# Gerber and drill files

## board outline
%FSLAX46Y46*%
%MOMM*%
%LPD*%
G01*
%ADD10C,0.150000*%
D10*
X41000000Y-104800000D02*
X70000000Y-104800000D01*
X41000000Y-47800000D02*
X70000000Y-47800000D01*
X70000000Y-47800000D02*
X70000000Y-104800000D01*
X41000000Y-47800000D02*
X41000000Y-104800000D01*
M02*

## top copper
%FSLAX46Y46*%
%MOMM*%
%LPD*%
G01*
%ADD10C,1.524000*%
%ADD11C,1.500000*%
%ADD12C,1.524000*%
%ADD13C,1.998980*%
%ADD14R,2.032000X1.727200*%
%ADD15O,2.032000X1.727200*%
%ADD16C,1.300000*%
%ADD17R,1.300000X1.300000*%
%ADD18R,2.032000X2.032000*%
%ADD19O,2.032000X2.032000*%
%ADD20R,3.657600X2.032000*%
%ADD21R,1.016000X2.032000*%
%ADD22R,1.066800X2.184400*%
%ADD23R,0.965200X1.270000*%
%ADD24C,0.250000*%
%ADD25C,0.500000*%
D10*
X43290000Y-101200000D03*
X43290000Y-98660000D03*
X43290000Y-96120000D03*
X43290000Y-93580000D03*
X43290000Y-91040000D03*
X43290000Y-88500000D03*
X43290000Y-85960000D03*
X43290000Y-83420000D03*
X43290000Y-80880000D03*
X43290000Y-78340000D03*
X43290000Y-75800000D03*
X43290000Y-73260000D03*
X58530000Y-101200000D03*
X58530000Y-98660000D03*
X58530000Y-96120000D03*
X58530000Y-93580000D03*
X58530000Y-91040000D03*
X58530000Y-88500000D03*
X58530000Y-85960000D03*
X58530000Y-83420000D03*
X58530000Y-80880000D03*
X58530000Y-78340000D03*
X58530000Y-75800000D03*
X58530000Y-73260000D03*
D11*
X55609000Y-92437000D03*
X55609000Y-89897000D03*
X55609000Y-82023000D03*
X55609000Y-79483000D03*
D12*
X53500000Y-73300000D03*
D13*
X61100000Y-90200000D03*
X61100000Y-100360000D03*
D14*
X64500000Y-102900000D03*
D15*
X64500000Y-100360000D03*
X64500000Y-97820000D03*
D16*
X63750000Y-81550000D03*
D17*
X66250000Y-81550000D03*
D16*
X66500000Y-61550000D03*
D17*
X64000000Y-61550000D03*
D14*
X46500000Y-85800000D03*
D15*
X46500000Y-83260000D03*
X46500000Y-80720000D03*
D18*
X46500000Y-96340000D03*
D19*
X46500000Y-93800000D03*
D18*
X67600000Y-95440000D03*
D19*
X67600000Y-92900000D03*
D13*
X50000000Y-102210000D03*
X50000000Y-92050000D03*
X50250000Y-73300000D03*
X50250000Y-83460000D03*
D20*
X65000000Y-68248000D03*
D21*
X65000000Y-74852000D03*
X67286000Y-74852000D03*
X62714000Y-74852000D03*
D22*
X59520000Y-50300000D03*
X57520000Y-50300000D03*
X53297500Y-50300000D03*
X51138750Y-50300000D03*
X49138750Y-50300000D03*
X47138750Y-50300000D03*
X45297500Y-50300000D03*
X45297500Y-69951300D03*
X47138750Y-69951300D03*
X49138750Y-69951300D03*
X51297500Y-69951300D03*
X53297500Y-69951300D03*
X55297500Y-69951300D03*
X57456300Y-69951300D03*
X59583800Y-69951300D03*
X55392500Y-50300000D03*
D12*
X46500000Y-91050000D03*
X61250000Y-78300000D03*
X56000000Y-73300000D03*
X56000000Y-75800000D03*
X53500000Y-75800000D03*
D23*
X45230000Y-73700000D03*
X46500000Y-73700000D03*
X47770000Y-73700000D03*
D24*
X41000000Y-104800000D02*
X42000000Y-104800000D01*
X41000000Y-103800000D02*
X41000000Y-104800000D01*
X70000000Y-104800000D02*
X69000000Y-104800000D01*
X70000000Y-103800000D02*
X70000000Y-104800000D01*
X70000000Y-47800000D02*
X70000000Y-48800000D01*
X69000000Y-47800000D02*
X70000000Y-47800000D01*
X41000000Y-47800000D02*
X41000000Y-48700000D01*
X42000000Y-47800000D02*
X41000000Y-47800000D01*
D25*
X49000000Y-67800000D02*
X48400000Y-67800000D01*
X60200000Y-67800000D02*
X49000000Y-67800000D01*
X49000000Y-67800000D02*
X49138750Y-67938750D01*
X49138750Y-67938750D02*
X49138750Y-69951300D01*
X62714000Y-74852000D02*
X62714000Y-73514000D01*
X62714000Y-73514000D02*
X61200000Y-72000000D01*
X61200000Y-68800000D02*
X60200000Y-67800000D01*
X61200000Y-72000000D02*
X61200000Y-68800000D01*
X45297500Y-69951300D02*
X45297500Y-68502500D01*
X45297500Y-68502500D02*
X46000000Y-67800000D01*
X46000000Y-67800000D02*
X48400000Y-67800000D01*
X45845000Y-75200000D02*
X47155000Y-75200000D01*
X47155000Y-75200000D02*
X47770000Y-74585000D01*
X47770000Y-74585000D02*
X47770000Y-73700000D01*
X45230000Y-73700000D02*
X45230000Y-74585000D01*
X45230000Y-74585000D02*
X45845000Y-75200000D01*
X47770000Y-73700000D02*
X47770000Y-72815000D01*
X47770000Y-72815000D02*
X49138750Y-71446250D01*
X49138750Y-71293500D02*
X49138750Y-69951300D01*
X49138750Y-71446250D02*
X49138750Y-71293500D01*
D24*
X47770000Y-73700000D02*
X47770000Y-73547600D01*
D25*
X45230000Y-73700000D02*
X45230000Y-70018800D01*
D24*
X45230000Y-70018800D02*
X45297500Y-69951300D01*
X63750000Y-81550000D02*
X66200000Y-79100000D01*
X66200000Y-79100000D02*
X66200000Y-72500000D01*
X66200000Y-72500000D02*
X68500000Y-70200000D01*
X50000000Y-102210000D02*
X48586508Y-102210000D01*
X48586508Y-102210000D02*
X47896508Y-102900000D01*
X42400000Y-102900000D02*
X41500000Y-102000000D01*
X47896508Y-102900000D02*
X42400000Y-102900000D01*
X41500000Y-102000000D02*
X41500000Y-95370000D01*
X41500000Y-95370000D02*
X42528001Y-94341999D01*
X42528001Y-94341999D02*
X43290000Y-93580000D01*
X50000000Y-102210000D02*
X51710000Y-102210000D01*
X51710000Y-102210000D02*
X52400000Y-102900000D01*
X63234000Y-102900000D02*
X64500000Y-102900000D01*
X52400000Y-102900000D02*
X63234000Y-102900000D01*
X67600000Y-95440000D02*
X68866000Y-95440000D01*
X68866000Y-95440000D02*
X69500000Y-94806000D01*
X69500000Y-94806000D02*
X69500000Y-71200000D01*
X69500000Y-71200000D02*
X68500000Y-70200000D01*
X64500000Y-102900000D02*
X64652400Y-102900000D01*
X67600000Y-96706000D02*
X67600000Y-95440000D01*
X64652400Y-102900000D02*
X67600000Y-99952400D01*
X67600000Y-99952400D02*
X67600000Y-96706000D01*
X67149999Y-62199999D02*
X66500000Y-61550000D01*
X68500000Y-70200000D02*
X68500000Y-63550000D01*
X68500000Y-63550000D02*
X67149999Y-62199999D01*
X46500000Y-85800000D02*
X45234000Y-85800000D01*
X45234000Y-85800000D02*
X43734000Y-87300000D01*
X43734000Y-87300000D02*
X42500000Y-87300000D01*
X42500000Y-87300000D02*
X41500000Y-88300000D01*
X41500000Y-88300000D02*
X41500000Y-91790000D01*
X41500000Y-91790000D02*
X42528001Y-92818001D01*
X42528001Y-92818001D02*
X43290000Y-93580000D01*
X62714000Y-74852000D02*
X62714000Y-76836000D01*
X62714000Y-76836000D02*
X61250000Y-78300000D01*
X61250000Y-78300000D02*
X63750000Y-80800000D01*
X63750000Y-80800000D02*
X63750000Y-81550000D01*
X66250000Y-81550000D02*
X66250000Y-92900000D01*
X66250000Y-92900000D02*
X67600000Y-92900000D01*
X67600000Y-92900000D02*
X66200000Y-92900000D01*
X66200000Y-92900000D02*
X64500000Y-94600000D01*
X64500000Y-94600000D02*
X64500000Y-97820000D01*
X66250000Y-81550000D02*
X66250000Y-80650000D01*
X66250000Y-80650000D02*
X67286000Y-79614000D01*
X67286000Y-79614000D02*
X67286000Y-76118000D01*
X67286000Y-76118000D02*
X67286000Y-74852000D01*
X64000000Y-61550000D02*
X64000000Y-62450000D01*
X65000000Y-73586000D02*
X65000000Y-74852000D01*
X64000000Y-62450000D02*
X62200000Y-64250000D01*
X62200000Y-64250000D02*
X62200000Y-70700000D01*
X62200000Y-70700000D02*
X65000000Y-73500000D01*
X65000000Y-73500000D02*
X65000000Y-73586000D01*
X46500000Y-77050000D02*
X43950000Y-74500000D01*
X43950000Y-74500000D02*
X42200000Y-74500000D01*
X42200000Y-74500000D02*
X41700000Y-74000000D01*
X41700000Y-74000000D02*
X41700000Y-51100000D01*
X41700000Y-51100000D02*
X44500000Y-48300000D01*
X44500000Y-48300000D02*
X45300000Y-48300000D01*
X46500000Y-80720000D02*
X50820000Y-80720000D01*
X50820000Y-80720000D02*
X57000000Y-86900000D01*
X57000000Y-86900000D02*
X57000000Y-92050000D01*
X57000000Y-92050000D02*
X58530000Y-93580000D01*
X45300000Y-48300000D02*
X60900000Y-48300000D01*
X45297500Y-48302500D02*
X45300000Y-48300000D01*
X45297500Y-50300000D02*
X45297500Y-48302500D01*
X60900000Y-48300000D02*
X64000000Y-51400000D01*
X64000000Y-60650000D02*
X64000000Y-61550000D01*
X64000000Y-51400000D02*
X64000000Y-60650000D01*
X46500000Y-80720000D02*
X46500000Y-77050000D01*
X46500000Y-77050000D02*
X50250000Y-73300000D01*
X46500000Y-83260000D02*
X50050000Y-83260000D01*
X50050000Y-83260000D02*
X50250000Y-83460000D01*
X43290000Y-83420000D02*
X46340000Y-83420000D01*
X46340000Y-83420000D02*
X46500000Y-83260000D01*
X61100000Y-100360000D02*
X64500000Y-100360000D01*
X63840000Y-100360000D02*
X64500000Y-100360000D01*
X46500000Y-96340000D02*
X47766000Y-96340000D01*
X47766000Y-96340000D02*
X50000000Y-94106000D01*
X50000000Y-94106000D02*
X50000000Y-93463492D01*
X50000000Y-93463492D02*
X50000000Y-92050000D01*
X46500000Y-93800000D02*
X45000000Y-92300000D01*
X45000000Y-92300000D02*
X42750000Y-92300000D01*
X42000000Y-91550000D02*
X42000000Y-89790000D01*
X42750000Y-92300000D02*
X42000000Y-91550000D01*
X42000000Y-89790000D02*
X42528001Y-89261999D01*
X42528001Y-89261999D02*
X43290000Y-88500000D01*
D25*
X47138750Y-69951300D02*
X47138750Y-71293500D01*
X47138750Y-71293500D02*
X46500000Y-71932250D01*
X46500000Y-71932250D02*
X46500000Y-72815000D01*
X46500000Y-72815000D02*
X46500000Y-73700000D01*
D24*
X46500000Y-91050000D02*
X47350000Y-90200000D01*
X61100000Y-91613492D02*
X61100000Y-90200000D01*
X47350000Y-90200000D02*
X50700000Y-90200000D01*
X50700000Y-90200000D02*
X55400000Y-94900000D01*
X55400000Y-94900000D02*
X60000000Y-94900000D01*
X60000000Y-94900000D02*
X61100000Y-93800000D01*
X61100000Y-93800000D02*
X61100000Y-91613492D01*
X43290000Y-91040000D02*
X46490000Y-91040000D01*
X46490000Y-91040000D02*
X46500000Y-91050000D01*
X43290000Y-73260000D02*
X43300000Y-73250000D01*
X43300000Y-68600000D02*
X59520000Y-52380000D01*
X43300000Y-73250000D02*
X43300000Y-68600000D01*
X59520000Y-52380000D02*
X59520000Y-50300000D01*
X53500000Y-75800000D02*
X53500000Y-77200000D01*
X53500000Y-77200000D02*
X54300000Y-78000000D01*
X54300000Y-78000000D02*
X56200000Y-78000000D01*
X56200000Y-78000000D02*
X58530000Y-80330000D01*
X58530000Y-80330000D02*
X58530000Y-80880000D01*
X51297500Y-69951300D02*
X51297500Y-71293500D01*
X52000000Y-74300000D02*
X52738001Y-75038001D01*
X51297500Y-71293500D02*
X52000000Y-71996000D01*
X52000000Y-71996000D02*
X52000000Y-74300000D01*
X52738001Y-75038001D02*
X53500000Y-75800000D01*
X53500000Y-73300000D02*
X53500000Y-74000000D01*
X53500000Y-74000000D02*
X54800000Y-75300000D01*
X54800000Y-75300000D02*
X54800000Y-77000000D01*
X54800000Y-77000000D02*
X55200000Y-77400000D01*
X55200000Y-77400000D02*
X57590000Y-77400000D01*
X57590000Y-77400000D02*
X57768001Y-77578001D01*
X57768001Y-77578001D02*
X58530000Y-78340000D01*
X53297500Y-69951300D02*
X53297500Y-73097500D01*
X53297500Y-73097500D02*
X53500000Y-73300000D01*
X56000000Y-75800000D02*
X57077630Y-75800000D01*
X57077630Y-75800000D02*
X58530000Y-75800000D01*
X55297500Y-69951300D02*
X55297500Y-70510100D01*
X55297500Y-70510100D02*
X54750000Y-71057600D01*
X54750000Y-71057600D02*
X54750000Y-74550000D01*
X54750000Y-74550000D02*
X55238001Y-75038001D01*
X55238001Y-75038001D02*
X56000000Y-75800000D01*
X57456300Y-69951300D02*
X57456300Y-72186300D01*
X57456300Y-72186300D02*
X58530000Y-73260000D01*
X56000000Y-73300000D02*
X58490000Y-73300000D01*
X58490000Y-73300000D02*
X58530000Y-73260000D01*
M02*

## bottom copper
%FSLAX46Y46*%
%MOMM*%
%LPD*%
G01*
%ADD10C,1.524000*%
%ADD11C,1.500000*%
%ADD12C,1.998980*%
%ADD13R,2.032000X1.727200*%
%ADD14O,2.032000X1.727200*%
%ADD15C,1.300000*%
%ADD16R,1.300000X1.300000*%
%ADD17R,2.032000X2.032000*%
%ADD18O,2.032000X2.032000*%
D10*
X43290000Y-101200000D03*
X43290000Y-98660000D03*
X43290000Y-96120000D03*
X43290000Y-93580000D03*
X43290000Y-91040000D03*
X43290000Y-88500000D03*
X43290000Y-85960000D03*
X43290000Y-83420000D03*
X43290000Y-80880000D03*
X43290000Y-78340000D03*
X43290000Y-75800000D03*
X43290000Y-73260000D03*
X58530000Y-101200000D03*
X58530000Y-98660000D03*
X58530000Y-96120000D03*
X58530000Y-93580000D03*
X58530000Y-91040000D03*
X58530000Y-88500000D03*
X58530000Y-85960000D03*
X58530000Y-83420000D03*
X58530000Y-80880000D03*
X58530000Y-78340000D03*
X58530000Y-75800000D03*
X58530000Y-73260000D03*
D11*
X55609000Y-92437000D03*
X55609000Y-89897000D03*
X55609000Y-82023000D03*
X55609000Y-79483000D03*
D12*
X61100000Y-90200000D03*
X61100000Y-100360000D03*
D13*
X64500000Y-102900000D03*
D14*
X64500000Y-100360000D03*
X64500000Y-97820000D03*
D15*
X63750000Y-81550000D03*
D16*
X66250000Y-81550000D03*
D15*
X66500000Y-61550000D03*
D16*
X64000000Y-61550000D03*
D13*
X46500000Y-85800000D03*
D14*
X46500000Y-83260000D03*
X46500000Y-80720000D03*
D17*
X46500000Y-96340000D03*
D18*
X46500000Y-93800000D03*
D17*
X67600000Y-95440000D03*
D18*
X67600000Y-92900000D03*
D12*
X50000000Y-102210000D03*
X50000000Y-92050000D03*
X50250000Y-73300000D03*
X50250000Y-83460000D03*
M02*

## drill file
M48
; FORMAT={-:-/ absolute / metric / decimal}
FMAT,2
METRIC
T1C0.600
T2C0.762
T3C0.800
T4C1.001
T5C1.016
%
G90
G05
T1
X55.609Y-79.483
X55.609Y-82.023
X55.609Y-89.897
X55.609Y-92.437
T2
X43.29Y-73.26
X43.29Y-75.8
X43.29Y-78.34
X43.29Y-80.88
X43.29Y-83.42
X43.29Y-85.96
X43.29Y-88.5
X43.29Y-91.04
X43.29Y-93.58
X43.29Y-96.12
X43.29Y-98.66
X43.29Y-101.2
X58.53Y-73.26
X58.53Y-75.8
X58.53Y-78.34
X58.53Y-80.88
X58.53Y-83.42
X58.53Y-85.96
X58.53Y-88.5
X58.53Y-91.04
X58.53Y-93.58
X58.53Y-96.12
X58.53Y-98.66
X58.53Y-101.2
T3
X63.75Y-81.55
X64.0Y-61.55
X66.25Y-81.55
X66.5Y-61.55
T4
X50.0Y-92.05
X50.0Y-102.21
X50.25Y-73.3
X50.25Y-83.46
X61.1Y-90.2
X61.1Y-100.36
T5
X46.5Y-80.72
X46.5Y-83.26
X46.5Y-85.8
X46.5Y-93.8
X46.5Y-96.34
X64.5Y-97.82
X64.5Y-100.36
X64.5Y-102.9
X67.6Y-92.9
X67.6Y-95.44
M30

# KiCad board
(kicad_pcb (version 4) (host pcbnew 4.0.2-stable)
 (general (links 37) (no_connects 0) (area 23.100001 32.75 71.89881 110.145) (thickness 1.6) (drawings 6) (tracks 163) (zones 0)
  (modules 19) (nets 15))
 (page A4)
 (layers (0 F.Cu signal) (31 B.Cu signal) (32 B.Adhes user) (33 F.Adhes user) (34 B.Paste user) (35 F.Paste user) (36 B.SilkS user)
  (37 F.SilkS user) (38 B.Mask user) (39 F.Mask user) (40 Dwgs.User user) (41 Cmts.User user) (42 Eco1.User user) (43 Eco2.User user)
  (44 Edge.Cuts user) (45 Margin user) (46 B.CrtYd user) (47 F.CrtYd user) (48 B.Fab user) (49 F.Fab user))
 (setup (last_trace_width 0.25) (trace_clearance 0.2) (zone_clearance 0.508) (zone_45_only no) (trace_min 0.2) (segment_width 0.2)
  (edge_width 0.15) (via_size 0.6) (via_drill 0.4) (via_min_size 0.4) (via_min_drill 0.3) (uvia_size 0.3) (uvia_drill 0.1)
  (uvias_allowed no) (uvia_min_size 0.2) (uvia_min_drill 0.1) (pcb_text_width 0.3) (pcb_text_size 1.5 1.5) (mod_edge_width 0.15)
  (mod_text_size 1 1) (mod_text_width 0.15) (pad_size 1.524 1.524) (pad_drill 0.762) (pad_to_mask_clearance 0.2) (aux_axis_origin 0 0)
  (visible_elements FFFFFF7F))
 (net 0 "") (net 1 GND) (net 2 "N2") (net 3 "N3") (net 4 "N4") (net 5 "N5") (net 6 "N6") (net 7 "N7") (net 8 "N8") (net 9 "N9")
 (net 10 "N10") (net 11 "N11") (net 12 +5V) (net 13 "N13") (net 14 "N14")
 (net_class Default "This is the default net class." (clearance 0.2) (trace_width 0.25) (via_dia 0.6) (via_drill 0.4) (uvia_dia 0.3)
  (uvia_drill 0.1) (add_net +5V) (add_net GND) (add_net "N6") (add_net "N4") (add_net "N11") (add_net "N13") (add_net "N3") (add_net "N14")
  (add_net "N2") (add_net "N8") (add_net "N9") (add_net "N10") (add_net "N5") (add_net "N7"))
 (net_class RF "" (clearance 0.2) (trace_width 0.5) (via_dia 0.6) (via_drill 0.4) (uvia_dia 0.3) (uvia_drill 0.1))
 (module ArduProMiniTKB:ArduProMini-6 (layer B.Cu) (at 40.75 107.55)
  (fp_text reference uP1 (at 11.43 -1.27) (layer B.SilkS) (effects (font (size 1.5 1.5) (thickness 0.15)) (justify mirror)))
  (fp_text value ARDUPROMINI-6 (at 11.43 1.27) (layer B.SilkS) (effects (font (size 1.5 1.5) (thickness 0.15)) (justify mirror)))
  (pad 7 thru_hole circle (at 2.54 -6.35) (size 1.524 1.524) (drill 0.762) (layers *.Cu *.Mask B.SilkS))
  (pad 8 thru_hole circle (at 2.54 -8.89) (size 1.524 1.524) (drill 0.762) (layers *.Cu *.Mask B.SilkS))
  (pad 9 thru_hole circle (at 2.54 -11.43) (size 1.524 1.524) (drill 0.762) (layers *.Cu *.Mask B.SilkS))
  (pad 10 thru_hole circle (at 2.54 -13.97) (size 1.524 1.524) (drill 0.762) (layers *.Cu *.Mask B.SilkS) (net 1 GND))
  (pad 11 thru_hole circle (at 2.54 -16.51) (size 1.524 1.524) (drill 0.762) (layers *.Cu *.Mask B.SilkS) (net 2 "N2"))
  (pad 12 thru_hole circle (at 2.54 -19.05) (size 1.524 1.524) (drill 0.762) (layers *.Cu *.Mask B.SilkS) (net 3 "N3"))
  (pad 13 thru_hole circle (at 2.54 -21.59) (size 1.524 1.524) (drill 0.762) (layers *.Cu *.Mask B.SilkS))
  (pad 14 thru_hole circle (at 2.54 -24.13) (size 1.524 1.524) (drill 0.762) (layers *.Cu *.Mask B.SilkS) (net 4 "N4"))
  (pad 15 thru_hole circle (at 2.54 -26.67) (size 1.524 1.524) (drill 0.762) (layers *.Cu *.Mask B.SilkS))
  (pad 16 thru_hole circle (at 2.54 -29.21) (size 1.524 1.524) (drill 0.762) (layers *.Cu *.Mask B.SilkS))
  (pad 17 thru_hole circle (at 2.54 -31.75) (size 1.524 1.524) (drill 0.762) (layers *.Cu *.Mask B.SilkS))
  (pad 18 thru_hole circle (at 2.54 -34.29) (size 1.524 1.524) (drill 0.762) (layers *.Cu *.Mask B.SilkS) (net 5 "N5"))
  (pad 19 thru_hole circle (at 17.78 -6.35) (size 1.524 1.524) (drill 0.762) (layers *.Cu *.Mask B.SilkS))
  (pad 20 thru_hole circle (at 17.78 -8.89) (size 1.524 1.524) (drill 0.762) (layers *.Cu *.Mask B.SilkS))
  (pad 21 thru_hole circle (at 17.78 -11.43) (size 1.524 1.524) (drill 0.762) (layers *.Cu *.Mask B.SilkS))
  (pad 22 thru_hole circle (at 17.78 -13.97) (size 1.524 1.524) (drill 0.762) (layers *.Cu *.Mask B.SilkS) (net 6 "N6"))
  (pad 23 thru_hole circle (at 17.78 -16.51) (size 1.524 1.524) (drill 0.762) (layers *.Cu *.Mask B.SilkS))
  (pad 24 thru_hole circle (at 17.78 -19.05) (size 1.524 1.524) (drill 0.762) (layers *.Cu *.Mask B.SilkS))
  (pad 25 thru_hole circle (at 17.78 -21.59) (size 1.524 1.524) (drill 0.762) (layers *.Cu *.Mask B.SilkS))
  (pad 26 thru_hole circle (at 17.78 -24.13) (size 1.524 1.524) (drill 0.762) (layers *.Cu *.Mask B.SilkS))
  (pad 27 thru_hole circle (at 17.78 -26.67) (size 1.524 1.524) (drill 0.762) (layers *.Cu *.Mask B.SilkS) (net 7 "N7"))
  (pad 28 thru_hole circle (at 17.78 -29.21) (size 1.524 1.524) (drill 0.762) (layers *.Cu *.Mask B.SilkS) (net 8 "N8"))
  (pad 29 thru_hole circle (at 17.78 -31.75) (size 1.524 1.524) (drill 0.762) (layers *.Cu *.Mask B.SilkS) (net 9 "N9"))
  (pad 30 thru_hole circle (at 17.78 -34.29) (size 1.524 1.524) (drill 0.762) (layers *.Cu *.Mask B.SilkS) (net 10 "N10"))
  (pad 31 thru_hole circle (at 14.859 -15.113) (size 1.5 1.5) (drill 0.6) (layers *.Cu *.Mask B.SilkS))
  (pad 32 thru_hole circle (at 14.859 -17.653) (size 1.5 1.5) (drill 0.6) (layers *.Cu *.Mask B.SilkS))
  (pad 34 thru_hole circle (at 14.859 -25.527) (size 1.5 1.5) (drill 0.6) (layers *.Cu *.Mask B.SilkS))
  (pad 35 thru_hole circle (at 14.859 -28.067) (size 1.5 1.5) (drill 0.6) (layers *.Cu *.Mask B.SilkS)))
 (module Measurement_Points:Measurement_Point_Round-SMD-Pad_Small (layer F.Cu) (at 53.5 73.3)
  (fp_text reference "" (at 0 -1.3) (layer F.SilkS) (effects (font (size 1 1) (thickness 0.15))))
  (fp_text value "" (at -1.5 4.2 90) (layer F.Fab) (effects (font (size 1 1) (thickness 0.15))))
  (pad 1 smd circle (at 0 0) (size 1.524 1.524) (layers F.Cu F.Paste F.Mask) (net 8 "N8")))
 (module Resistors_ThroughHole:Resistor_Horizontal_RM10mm (layer F.Cu) (at 61.1 90.2 270)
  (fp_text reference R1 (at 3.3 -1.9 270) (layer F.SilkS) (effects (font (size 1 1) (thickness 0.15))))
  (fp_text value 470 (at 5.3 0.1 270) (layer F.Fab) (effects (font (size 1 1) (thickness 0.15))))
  (pad 1 thru_hole circle (at 0 0 270) (size 1.99898 1.99898) (drill 1.00076) (layers *.Cu *.SilkS *.Mask) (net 2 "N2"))
  (pad 2 thru_hole circle (at 10.16 0 270) (size 1.99898 1.99898) (drill 1.00076) (layers *.Cu *.SilkS *.Mask) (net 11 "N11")))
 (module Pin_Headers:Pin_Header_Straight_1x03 (layer F.Cu) (at 64.5 102.9 180)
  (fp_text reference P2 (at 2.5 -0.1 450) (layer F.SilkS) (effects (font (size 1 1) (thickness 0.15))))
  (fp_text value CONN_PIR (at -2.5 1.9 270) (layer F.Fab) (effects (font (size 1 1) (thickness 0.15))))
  (pad 1 thru_hole rect (at 0 0 180) (size 2.032 1.7272) (drill 1.016) (layers *.Cu *.Mask F.SilkS) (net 1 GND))
  (pad 2 thru_hole oval (at 0 2.54 180) (size 2.032 1.7272) (drill 1.016) (layers *.Cu *.Mask F.SilkS) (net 11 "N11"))
  (pad 3 thru_hole oval (at 0 5.08 180) (size 2.032 1.7272) (drill 1.016) (layers *.Cu *.Mask F.SilkS) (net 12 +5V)))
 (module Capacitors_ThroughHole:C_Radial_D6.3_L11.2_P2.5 (layer F.Cu) (at 66.25 81.55 180)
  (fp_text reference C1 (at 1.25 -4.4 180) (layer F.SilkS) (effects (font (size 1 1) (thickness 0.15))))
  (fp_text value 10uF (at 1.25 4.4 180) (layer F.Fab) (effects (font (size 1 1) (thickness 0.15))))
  (pad 2 thru_hole circle (at 2.5 0 180) (size 1.3 1.3) (drill 0.8) (layers *.Cu *.Mask F.SilkS) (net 1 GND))
  (pad 1 thru_hole rect (at 0 0 180) (size 1.3 1.3) (drill 0.8) (layers *.Cu *.Mask F.SilkS) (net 12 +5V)))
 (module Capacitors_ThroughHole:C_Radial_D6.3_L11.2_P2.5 (layer F.Cu) (at 64 61.55)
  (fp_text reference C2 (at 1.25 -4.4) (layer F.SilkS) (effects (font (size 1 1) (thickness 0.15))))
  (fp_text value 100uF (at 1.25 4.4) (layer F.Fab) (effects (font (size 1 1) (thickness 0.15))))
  (pad 2 thru_hole circle (at 2.5 0) (size 1.3 1.3) (drill 0.8) (layers *.Cu *.Mask F.SilkS) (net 1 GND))
  (pad 1 thru_hole rect (at 0 0) (size 1.3 1.3) (drill 0.8) (layers *.Cu *.Mask F.SilkS) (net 6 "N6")))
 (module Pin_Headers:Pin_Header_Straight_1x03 (layer F.Cu) (at 46.5 85.8 180)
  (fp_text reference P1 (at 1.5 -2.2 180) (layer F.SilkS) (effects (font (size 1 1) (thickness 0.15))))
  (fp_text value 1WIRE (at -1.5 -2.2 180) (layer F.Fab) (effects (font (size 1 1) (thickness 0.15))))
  (pad 1 thru_hole rect (at 0 0 180) (size 2.032 1.7272) (drill 1.016) (layers *.Cu *.Mask F.SilkS) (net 1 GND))
  (pad 2 thru_hole oval (at 0 2.54 180) (size 2.032 1.7272) (drill 1.016) (layers *.Cu *.Mask F.SilkS) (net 4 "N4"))
  (pad 3 thru_hole oval (at 0 5.08 180) (size 2.032 1.7272) (drill 1.016) (layers *.Cu *.Mask F.SilkS) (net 6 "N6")))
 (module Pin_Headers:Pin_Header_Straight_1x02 (layer F.Cu) (at 46.5 96.34 180)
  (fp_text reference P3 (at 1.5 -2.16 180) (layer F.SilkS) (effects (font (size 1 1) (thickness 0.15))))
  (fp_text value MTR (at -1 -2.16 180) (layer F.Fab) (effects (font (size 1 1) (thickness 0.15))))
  (pad 1 thru_hole rect (at 0 0 180) (size 2.032 2.032) (drill 1.016) (layers *.Cu *.Mask F.SilkS) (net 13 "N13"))
  (pad 2 thru_hole oval (at 0 2.54 180) (size 2.032 2.032) (drill 1.016) (layers *.Cu *.Mask F.SilkS) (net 3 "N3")))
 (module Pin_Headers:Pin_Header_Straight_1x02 (layer F.Cu) (at 67.6 95.44 180)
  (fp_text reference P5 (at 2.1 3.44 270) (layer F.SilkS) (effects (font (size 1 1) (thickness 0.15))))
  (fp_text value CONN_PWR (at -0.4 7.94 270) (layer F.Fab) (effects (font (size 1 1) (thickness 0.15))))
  (pad 1 thru_hole rect (at 0 0 180) (size 2.032 2.032) (drill 1.016) (layers *.Cu *.Mask F.SilkS) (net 1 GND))
  (pad 2 thru_hole oval (at 0 2.54 180) (size 2.032 2.032) (drill 1.016) (layers *.Cu *.Mask F.SilkS) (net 12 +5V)))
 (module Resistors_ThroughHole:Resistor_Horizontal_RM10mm (layer F.Cu) (at 50 102.21 90)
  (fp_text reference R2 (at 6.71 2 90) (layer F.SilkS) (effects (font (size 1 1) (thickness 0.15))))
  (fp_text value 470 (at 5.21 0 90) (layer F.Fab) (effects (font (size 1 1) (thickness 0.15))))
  (pad 1 thru_hole circle (at 0 0 90) (size 1.99898 1.99898) (drill 1.00076) (layers *.Cu *.SilkS *.Mask) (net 1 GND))
  (pad 2 thru_hole circle (at 10.16 0 90) (size 1.99898 1.99898) (drill 1.00076) (layers *.Cu *.SilkS *.Mask) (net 13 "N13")))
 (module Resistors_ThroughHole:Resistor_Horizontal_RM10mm (layer F.Cu) (at 50.25 73.3 270)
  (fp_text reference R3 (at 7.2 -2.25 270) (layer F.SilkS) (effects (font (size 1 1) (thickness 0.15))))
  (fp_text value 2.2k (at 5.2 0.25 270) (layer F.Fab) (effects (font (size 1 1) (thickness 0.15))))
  (pad 1 thru_hole circle (at 0 0 270) (size 1.99898 1.99898) (drill 1.00076) (layers *.Cu *.SilkS *.Mask) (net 6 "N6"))
  (pad 2 thru_hole circle (at 10.16 0 270) (size 1.99898 1.99898) (drill 1.00076) (layers *.Cu *.SilkS *.Mask) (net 4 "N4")))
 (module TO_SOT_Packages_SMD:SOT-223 (layer F.Cu) (at 65 71.55)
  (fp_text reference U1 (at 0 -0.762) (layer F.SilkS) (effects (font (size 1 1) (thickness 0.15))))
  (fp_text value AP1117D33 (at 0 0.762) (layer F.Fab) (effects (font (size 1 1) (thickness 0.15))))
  (pad 4 smd rect (at 0 -3.302) (size 3.6576 2.032) (layers F.Cu F.Paste F.Mask))
  (pad 2 smd rect (at 0 3.302) (size 1.016 2.032) (layers F.Cu F.Paste F.Mask) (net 6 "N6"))
  (pad 3 smd rect (at 2.286 3.302) (size 1.016 2.032) (layers F.Cu F.Paste F.Mask) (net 12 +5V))
  (pad 1 smd rect (at -2.286 3.302) (size 1.016 2.032) (layers F.Cu F.Paste F.Mask) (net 1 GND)))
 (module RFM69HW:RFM (layer F.Cu) (at 44.25 50.3 270) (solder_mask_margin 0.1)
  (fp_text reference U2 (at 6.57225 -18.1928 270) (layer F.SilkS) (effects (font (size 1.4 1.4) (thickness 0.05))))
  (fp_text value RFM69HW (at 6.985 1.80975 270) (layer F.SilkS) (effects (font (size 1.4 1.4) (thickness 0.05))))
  (pad RESE smd rect (at 0 -15.27 270) (size 2.1844 1.0668) (layers F.Cu F.Paste F.Mask) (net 5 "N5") (solder_mask_margin 0.2))
  (pad DIO0 smd rect (at 0 -13.27 270) (size 2.1844 1.0668) (layers F.Cu F.Paste F.Mask) (solder_mask_margin 0.2))
  (pad DIO2 smd rect (at 0 -9.0475 270) (size 2.1844 1.0668) (layers F.Cu F.Paste F.Mask) (solder_mask_margin 0.2))
  (pad DIO3 smd rect (at 0 -6.88875 270) (size 2.1844 1.0668) (layers F.Cu F.Paste F.Mask) (solder_mask_margin 0.2))
  (pad DIO4 smd rect (at 0 -4.88875 270) (size 2.1844 1.0668) (layers F.Cu F.Paste F.Mask) (solder_mask_margin 0.2))
  (pad DIO5 smd rect (at 0 -2.88875 270) (size 2.1844 1.0668) (layers F.Cu F.Paste F.Mask) (solder_mask_margin 0.2))
  (pad VCC smd rect (at 0 -1.0475 270) (size 2.1844 1.0668) (layers F.Cu F.Paste F.Mask) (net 6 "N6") (solder_mask_margin 0.2))
  (pad GNDB smd rect (at 19.6513 -1.0475 270) (size 2.1844 1.0668) (layers F.Cu F.Paste F.Mask) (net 1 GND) (solder_mask_margin 0.2))
  (pad ANT smd rect (at 19.6513 -2.88875 270) (size 2.1844 1.0668) (layers F.Cu F.Paste F.Mask) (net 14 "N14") (solder_mask_margin 0.2))
  (pad GNDA smd rect (at 19.6513 -4.88875 270) (size 2.1844 1.0668) (layers F.Cu F.Paste F.Mask) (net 1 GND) (solder_mask_margin 0.2))
  (pad SCK smd rect (at 19.6513 -7.0475 270) (size 2.1844 1.0668) (layers F.Cu F.Paste F.Mask) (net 7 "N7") (solder_mask_margin 0.2))
  (pad MISO smd rect (at 19.6513 -9.0475 270) (size 2.1844 1.0668) (layers F.Cu F.Paste F.Mask) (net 8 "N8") (solder_mask_margin 0.2))
  (pad MOSI smd rect (at 19.6513 -11.0475 270) (size 2.1844 1.0668) (layers F.Cu F.Paste F.Mask) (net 9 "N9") (solder_mask_margin 0.2))
  (pad NSS smd rect (at 19.6513 -13.2063 270) (size 2.1844 1.0668) (layers F.Cu F.Paste F.Mask) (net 10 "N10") (solder_mask_margin 0.2))
  (pad NC smd rect (at 19.6513 -15.3338 270) (size 2.1844 1.0668) (layers F.Cu F.Paste F.Mask) (solder_mask_margin 0.2))
  (pad DIO1 smd rect (at 0 -11.1425 270) (size 2.1844 1.0668) (layers F.Cu F.Paste F.Mask) (solder_mask_margin 0.2)))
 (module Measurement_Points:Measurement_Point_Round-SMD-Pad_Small (layer F.Cu) (at 46.5 91.05)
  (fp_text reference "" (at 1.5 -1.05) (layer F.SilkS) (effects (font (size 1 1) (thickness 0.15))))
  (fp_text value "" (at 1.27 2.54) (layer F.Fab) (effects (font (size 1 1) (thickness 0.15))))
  (pad 1 smd circle (at 0 0) (size 1.524 1.524) (layers F.Cu F.Paste F.Mask) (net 2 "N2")))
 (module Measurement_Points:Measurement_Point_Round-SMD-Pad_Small (layer F.Cu) (at 61.25 78.3)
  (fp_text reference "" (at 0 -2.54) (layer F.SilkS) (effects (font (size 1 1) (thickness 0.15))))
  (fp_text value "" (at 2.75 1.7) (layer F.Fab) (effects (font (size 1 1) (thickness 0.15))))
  (pad 1 smd circle (at 0 0) (size 1.524 1.524) (layers F.Cu F.Paste F.Mask) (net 1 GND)))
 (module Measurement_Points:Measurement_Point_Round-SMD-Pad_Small (layer F.Cu) (at 56 73.3)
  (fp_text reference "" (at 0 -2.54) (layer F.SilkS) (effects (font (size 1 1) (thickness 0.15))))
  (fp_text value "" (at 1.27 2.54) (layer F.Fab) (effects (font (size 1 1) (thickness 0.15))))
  (pad 1 smd circle (at 0 0) (size 1.524 1.524) (layers F.Cu F.Paste F.Mask) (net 10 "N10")))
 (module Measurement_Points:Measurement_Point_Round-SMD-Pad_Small (layer F.Cu) (at 56 75.8)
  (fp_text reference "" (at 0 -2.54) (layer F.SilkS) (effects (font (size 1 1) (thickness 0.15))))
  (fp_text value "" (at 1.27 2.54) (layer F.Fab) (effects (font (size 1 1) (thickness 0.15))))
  (pad 1 smd circle (at 0 0) (size 1.524 1.524) (layers F.Cu F.Paste F.Mask) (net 9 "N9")))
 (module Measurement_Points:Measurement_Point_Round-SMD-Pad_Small (layer F.Cu) (at 53.5 75.8)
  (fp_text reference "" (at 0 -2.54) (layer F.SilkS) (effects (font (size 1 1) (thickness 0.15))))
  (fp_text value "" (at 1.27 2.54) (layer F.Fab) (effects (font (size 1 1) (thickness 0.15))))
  (pad 1 smd circle (at 0 0) (size 1.524 1.524) (layers F.Cu F.Paste F.Mask) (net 7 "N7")))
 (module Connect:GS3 (layer F.Cu) (at 46.5 73.7 90)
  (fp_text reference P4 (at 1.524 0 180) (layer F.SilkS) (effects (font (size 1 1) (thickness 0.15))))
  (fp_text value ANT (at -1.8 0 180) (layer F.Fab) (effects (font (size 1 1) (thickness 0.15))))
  (pad 1 smd rect (at 0 -1.27 90) (size 1.27 0.9652) (layers F.Cu F.Paste F.Mask) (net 1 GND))
  (pad 2 smd rect (at 0 0 90) (size 1.27 0.9652) (layers F.Cu F.Paste F.Mask) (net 14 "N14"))
  (pad 3 smd rect (at 0 1.27 90) (size 1.27 0.9652) (layers F.Cu F.Paste F.Mask) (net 1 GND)))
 (gr_line (start 41 104.8) (end 70 104.8) (angle 90) (layer Edge.Cuts) (width 0.15))
 (gr_line (start 41 47.8) (end 70 47.8) (angle 90) (layer Edge.Cuts) (width 0.15))
 (gr_line (start 70 47.8) (end 70 104.8) (angle 90) (layer Edge.Cuts) (width 0.15))
 (gr_line (start 41 47.8) (end 41 104.8) (angle 90) (layer Edge.Cuts) (width 0.15))
 (segment (start 41 104.8) (end 42 104.8) (width 0.25) (layer F.Cu) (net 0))
 (segment (start 41 103.8) (end 41 104.8) (width 0.25) (layer F.Cu) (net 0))
 (segment (start 70 104.8) (end 69 104.8) (width 0.25) (layer F.Cu) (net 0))
 (segment (start 70 103.8) (end 70 104.8) (width 0.25) (layer F.Cu) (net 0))
 (segment (start 70 47.8) (end 70 48.8) (width 0.25) (layer F.Cu) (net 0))
 (segment (start 69 47.8) (end 70 47.8) (width 0.25) (layer F.Cu) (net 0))
 (segment (start 41 47.8) (end 41 48.7) (width 0.25) (layer F.Cu) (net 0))
 (segment (start 42 47.8) (end 41 47.8) (width 0.25) (layer F.Cu) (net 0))
 (segment (start 49 67.8) (end 48.4 67.8) (width 0.5) (layer F.Cu) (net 1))
 (segment (start 60.2 67.8) (end 49 67.8) (width 0.5) (layer F.Cu) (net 1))
 (segment (start 49 67.8) (end 49.13875 67.93875) (width 0.5) (layer F.Cu) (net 1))
 (segment (start 49.13875 67.93875) (end 49.13875 69.9513) (width 0.5) (layer F.Cu) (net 1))
 (segment (start 62.714 74.852) (end 62.714 73.514) (width 0.5) (layer F.Cu) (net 1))
 (segment (start 62.714 73.514) (end 61.2 72) (width 0.5) (layer F.Cu) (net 1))
 (segment (start 61.2 68.8) (end 60.2 67.8) (width 0.5) (layer F.Cu) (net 1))
 (segment (start 61.2 72) (end 61.2 68.8) (width 0.5) (layer F.Cu) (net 1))
 (segment (start 45.2975 69.9513) (end 45.2975 68.5025) (width 0.5) (layer F.Cu) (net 1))
 (segment (start 45.2975 68.5025) (end 46 67.8) (width 0.5) (layer F.Cu) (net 1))
 (segment (start 46 67.8) (end 48.4 67.8) (width 0.5) (layer F.Cu) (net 1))
 (segment (start 45.845 75.2) (end 47.155 75.2) (width 0.5) (layer F.Cu) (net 1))
 (segment (start 47.155 75.2) (end 47.77 74.585) (width 0.5) (layer F.Cu) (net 1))
 (segment (start 47.77 74.585) (end 47.77 73.7) (width 0.5) (layer F.Cu) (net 1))
 (segment (start 45.23 73.7) (end 45.23 74.585) (width 0.5) (layer F.Cu) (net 1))
 (segment (start 45.23 74.585) (end 45.845 75.2) (width 0.5) (layer F.Cu) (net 1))
 (segment (start 47.77 73.7) (end 47.77 72.815) (width 0.5) (layer F.Cu) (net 1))
 (segment (start 47.77 72.815) (end 49.13875 71.44625) (width 0.5) (layer F.Cu) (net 1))
 (segment (start 49.13875 71.2935) (end 49.13875 69.9513) (width 0.5) (layer F.Cu) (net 1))
 (segment (start 49.13875 71.44625) (end 49.13875 71.2935) (width 0.5) (layer F.Cu) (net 1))
 (segment (start 47.77 73.7) (end 47.77 73.5476) (width 0.25) (layer F.Cu) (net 1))
 (segment (start 45.23 73.7) (end 45.23 70.0188) (width 0.5) (layer F.Cu) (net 1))
 (segment (start 45.23 70.0188) (end 45.2975 69.9513) (width 0.25) (layer F.Cu) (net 1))
 (segment (start 63.75 81.55) (end 66.2 79.1) (width 0.25) (layer F.Cu) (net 1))
 (segment (start 66.2 79.1) (end 66.2 72.5) (width 0.25) (layer F.Cu) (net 1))
 (segment (start 66.2 72.5) (end 68.5 70.2) (width 0.25) (layer F.Cu) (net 1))
 (segment (start 50 102.21) (end 48.586508 102.21) (width 0.25) (layer F.Cu) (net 1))
 (segment (start 48.586508 102.21) (end 47.896508 102.9) (width 0.25) (layer F.Cu) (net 1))
 (segment (start 42.4 102.9) (end 41.5 102) (width 0.25) (layer F.Cu) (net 1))
 (segment (start 47.896508 102.9) (end 42.4 102.9) (width 0.25) (layer F.Cu) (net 1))
 (segment (start 41.5 102) (end 41.5 95.37) (width 0.25) (layer F.Cu) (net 1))
 (segment (start 41.5 95.37) (end 42.528001 94.341999) (width 0.25) (layer F.Cu) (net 1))
 (segment (start 42.528001 94.341999) (end 43.29 93.58) (width 0.25) (layer F.Cu) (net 1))
 (segment (start 50 102.21) (end 51.71 102.21) (width 0.25) (layer F.Cu) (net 1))
 (segment (start 51.71 102.21) (end 52.4 102.9) (width 0.25) (layer F.Cu) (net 1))
 (segment (start 63.234 102.9) (end 64.5 102.9) (width 0.25) (layer F.Cu) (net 1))
 (segment (start 52.4 102.9) (end 63.234 102.9) (width 0.25) (layer F.Cu) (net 1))
 (segment (start 67.6 95.44) (end 68.866 95.44) (width 0.25) (layer F.Cu) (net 1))
 (segment (start 68.866 95.44) (end 69.5 94.806) (width 0.25) (layer F.Cu) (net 1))
 (segment (start 69.5 94.806) (end 69.5 71.2) (width 0.25) (layer F.Cu) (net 1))
 (segment (start 69.5 71.2) (end 68.5 70.2) (width 0.25) (layer F.Cu) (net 1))
 (segment (start 64.5 102.9) (end 64.6524 102.9) (width 0.25) (layer F.Cu) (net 1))
 (segment (start 67.6 96.706) (end 67.6 95.44) (width 0.25) (layer F.Cu) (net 1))
 (segment (start 64.6524 102.9) (end 67.6 99.9524) (width 0.25) (layer F.Cu) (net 1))
 (segment (start 67.6 99.9524) (end 67.6 96.706) (width 0.25) (layer F.Cu) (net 1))
 (segment (start 67.149999 62.199999) (end 66.5 61.55) (width 0.25) (layer F.Cu) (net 1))
 (segment (start 68.5 70.2) (end 68.5 63.55) (width 0.25) (layer F.Cu) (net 1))
 (segment (start 68.5 63.55) (end 67.149999 62.199999) (width 0.25) (layer F.Cu) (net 1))
 (segment (start 46.5 85.8) (end 45.234 85.8) (width 0.25) (layer F.Cu) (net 1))
 (segment (start 45.234 85.8) (end 43.734 87.3) (width 0.25) (layer F.Cu) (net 1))
 (segment (start 43.734 87.3) (end 42.5 87.3) (width 0.25) (layer F.Cu) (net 1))
 (segment (start 42.5 87.3) (end 41.5 88.3) (width 0.25) (layer F.Cu) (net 1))
 (segment (start 41.5 88.3) (end 41.5 91.79) (width 0.25) (layer F.Cu) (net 1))
 (segment (start 41.5 91.79) (end 42.528001 92.818001) (width 0.25) (layer F.Cu) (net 1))
 (segment (start 42.528001 92.818001) (end 43.29 93.58) (width 0.25) (layer F.Cu) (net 1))
 (segment (start 62.714 74.852) (end 62.714 76.836) (width 0.25) (layer F.Cu) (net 1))
 (segment (start 62.714 76.836) (end 61.25 78.3) (width 0.25) (layer F.Cu) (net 1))
 (segment (start 61.25 78.3) (end 63.75 80.8) (width 0.25) (layer F.Cu) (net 1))
 (segment (start 63.75 80.8) (end 63.75 81.55) (width 0.25) (layer F.Cu) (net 1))
 (segment (start 66.25 81.55) (end 66.25 92.9) (width 0.25) (layer F.Cu) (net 12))
 (segment (start 66.25 92.9) (end 67.6 92.9) (width 0.25) (layer F.Cu) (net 12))
 (segment (start 67.6 92.9) (end 66.2 92.9) (width 0.25) (layer F.Cu) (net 12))
 (segment (start 66.2 92.9) (end 64.5 94.6) (width 0.25) (layer F.Cu) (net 12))
 (segment (start 64.5 94.6) (end 64.5 97.82) (width 0.25) (layer F.Cu) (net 12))
 (segment (start 66.25 81.55) (end 66.25 80.65) (width 0.25) (layer F.Cu) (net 12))
 (segment (start 66.25 80.65) (end 67.286 79.614) (width 0.25) (layer F.Cu) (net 12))
 (segment (start 67.286 79.614) (end 67.286 76.118) (width 0.25) (layer F.Cu) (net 12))
 (segment (start 67.286 76.118) (end 67.286 74.852) (width 0.25) (layer F.Cu) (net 12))
 (segment (start 64 61.55) (end 64 62.45) (width 0.25) (layer F.Cu) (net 6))
 (segment (start 65 73.586) (end 65 74.852) (width 0.25) (layer F.Cu) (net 6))
 (segment (start 64 62.45) (end 62.2 64.25) (width 0.25) (layer F.Cu) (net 6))
 (segment (start 62.2 64.25) (end 62.2 70.7) (width 0.25) (layer F.Cu) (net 6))
 (segment (start 62.2 70.7) (end 65 73.5) (width 0.25) (layer F.Cu) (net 6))
 (segment (start 65 73.5) (end 65 73.586) (width 0.25) (layer F.Cu) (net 6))
 (segment (start 46.5 77.05) (end 43.95 74.5) (width 0.25) (layer F.Cu) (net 6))
 (segment (start 43.95 74.5) (end 42.2 74.5) (width 0.25) (layer F.Cu) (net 6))
 (segment (start 42.2 74.5) (end 41.7 74) (width 0.25) (layer F.Cu) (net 6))
 (segment (start 41.7 74) (end 41.7 51.1) (width 0.25) (layer F.Cu) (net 6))
 (segment (start 41.7 51.1) (end 44.5 48.3) (width 0.25) (layer F.Cu) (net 6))
 (segment (start 44.5 48.3) (end 45.3 48.3) (width 0.25) (layer F.Cu) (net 6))
 (segment (start 46.5 80.72) (end 50.82 80.72) (width 0.25) (layer F.Cu) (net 6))
 (segment (start 50.82 80.72) (end 57 86.9) (width 0.25) (layer F.Cu) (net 6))
 (segment (start 57 86.9) (end 57 92.05) (width 0.25) (layer F.Cu) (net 6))
 (segment (start 57 92.05) (end 58.53 93.58) (width 0.25) (layer F.Cu) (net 6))
 (segment (start 45.3 48.3) (end 60.9 48.3) (width 0.25) (layer F.Cu) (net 6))
 (segment (start 45.2975 48.3025) (end 45.3 48.3) (width 0.25) (layer F.Cu) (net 6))
 (segment (start 45.2975 50.3) (end 45.2975 48.3025) (width 0.25) (layer F.Cu) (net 6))
 (segment (start 60.9 48.3) (end 64 51.4) (width 0.25) (layer F.Cu) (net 6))
 (segment (start 64 60.65) (end 64 61.55) (width 0.25) (layer F.Cu) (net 6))
 (segment (start 64 51.4) (end 64 60.65) (width 0.25) (layer F.Cu) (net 6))
 (segment (start 46.5 80.72) (end 46.5 77.05) (width 0.25) (layer F.Cu) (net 6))
 (segment (start 46.5 77.05) (end 50.25 73.3) (width 0.25) (layer F.Cu) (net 6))
 (segment (start 46.5 83.26) (end 50.05 83.26) (width 0.25) (layer F.Cu) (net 4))
 (segment (start 50.05 83.26) (end 50.25 83.46) (width 0.25) (layer F.Cu) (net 4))
 (segment (start 43.29 83.42) (end 46.34 83.42) (width 0.25) (layer F.Cu) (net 4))
 (segment (start 46.34 83.42) (end 46.5 83.26) (width 0.25) (layer F.Cu) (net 4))
 (segment (start 61.1 100.36) (end 64.5 100.36) (width 0.25) (layer F.Cu) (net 11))
 (segment (start 63.84 100.36) (end 64.5 100.36) (width 0.25) (layer F.Cu) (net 11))
 (segment (start 46.5 96.34) (end 47.766 96.34) (width 0.25) (layer F.Cu) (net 13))
 (segment (start 47.766 96.34) (end 50 94.106) (width 0.25) (layer F.Cu) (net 13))
 (segment (start 50 94.106) (end 50 93.463492) (width 0.25) (layer F.Cu) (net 13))
 (segment (start 50 93.463492) (end 50 92.05) (width 0.25) (layer F.Cu) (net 13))
 (segment (start 46.5 93.8) (end 45 92.3) (width 0.25) (layer F.Cu) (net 3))
 (segment (start 45 92.3) (end 42.75 92.3) (width 0.25) (layer F.Cu) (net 3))
 (segment (start 42 91.55) (end 42 89.79) (width 0.25) (layer F.Cu) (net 3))
 (segment (start 42.75 92.3) (end 42 91.55) (width 0.25) (layer F.Cu) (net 3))
 (segment (start 42 89.79) (end 42.528001 89.261999) (width 0.25) (layer F.Cu) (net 3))
 (segment (start 42.528001 89.261999) (end 43.29 88.5) (width 0.25) (layer F.Cu) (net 3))
 (segment (start 47.13875 69.9513) (end 47.13875 71.2935) (width 0.5) (layer F.Cu) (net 14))
 (segment (start 47.13875 71.2935) (end 46.5 71.93225) (width 0.5) (layer F.Cu) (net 14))
 (segment (start 46.5 71.93225) (end 46.5 72.815) (width 0.5) (layer F.Cu) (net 14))
 (segment (start 46.5 72.815) (end 46.5 73.7) (width 0.5) (layer F.Cu) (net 14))
 (segment (start 46.5 91.05) (end 47.35 90.2) (width 0.25) (layer F.Cu) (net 2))
 (segment (start 61.1 91.613492) (end 61.1 90.2) (width 0.25) (layer F.Cu) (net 2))
 (segment (start 47.35 90.2) (end 50.7 90.2) (width 0.25) (layer F.Cu) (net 2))
 (segment (start 50.7 90.2) (end 55.4 94.9) (width 0.25) (layer F.Cu) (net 2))
 (segment (start 55.4 94.9) (end 60 94.9) (width 0.25) (layer F.Cu) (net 2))
 (segment (start 60 94.9) (end 61.1 93.8) (width 0.25) (layer F.Cu) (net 2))
 (segment (start 61.1 93.8) (end 61.1 91.613492) (width 0.25) (layer F.Cu) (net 2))
 (segment (start 43.29 91.04) (end 46.49 91.04) (width 0.25) (layer F.Cu) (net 2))
 (segment (start 46.49 91.04) (end 46.5 91.05) (width 0.25) (layer F.Cu) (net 2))
 (segment (start 43.29 73.26) (end 43.3 73.25) (width 0.25) (layer F.Cu) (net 5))
 (segment (start 43.3 68.6) (end 59.52 52.38) (width 0.25) (layer F.Cu) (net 5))
 (segment (start 43.3 73.25) (end 43.3 68.6) (width 0.25) (layer F.Cu) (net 5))
 (segment (start 59.52 52.38) (end 59.52 50.3) (width 0.25) (layer F.Cu) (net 5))
 (segment (start 53.5 75.8) (end 53.5 77.2) (width 0.25) (layer F.Cu) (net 7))
 (segment (start 53.5 77.2) (end 54.3 78) (width 0.25) (layer F.Cu) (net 7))
 (segment (start 54.3 78) (end 56.2 78) (width 0.25) (layer F.Cu) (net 7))
 (segment (start 56.2 78) (end 58.53 80.33) (width 0.25) (layer F.Cu) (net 7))
 (segment (start 58.53 80.33) (end 58.53 80.88) (width 0.25) (layer F.Cu) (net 7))
 (segment (start 51.2975 69.9513) (end 51.2975 71.2935) (width 0.25) (layer F.Cu) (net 7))
 (segment (start 52 74.3) (end 52.738001 75.038001) (width 0.25) (layer F.Cu) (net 7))
 (segment (start 51.2975 71.2935) (end 52 71.996) (width 0.25) (layer F.Cu) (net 7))
 (segment (start 52 71.996) (end 52 74.3) (width 0.25) (layer F.Cu) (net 7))
 (segment (start 52.738001 75.038001) (end 53.5 75.8) (width 0.25) (layer F.Cu) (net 7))
 (segment (start 53.5 73.3) (end 53.5 74) (width 0.25) (layer F.Cu) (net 8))
 (segment (start 53.5 74) (end 54.8 75.3) (width 0.25) (layer F.Cu) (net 8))
 (segment (start 54.8 75.3) (end 54.8 77) (width 0.25) (layer F.Cu) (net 8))
 (segment (start 54.8 77) (end 55.2 77.4) (width 0.25) (layer F.Cu) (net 8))
 (segment (start 55.2 77.4) (end 57.59 77.4) (width 0.25) (layer F.Cu) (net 8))
 (segment (start 57.59 77.4) (end 57.768001 77.578001) (width 0.25) (layer F.Cu) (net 8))
 (segment (start 57.768001 77.578001) (end 58.53 78.34) (width 0.25) (layer F.Cu) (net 8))
 (segment (start 53.2975 69.9513) (end 53.2975 73.0975) (width 0.25) (layer F.Cu) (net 8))
 (segment (start 53.2975 73.0975) (end 53.5 73.3) (width 0.25) (layer F.Cu) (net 8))
 (segment (start 56 75.8) (end 57.07763 75.8) (width 0.25) (layer F.Cu) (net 9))
 (segment (start 57.07763 75.8) (end 58.53 75.8) (width 0.25) (layer F.Cu) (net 9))
 (segment (start 55.2975 69.9513) (end 55.2975 70.5101) (width 0.25) (layer F.Cu) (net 9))
 (segment (start 55.2975 70.5101) (end 54.75 71.0576) (width 0.25) (layer F.Cu) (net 9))
 (segment (start 54.75 71.0576) (end 54.75 74.55) (width 0.25) (layer F.Cu) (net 9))
 (segment (start 54.75 74.55) (end 55.238001 75.038001) (width 0.25) (layer F.Cu) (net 9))
 (segment (start 55.238001 75.038001) (end 56 75.8) (width 0.25) (layer F.Cu) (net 9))
 (segment (start 57.4563 69.9513) (end 57.4563 72.1863) (width 0.25) (layer F.Cu) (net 10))
 (segment (start 57.4563 72.1863) (end 58.53 73.26) (width 0.25) (layer F.Cu) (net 10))
 (segment (start 56 73.3) (end 58.49 73.3) (width 0.25) (layer F.Cu) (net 10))
 (segment (start 58.49 73.3) (end 58.53 73.26) (width 0.25) (layer F.Cu) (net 10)))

